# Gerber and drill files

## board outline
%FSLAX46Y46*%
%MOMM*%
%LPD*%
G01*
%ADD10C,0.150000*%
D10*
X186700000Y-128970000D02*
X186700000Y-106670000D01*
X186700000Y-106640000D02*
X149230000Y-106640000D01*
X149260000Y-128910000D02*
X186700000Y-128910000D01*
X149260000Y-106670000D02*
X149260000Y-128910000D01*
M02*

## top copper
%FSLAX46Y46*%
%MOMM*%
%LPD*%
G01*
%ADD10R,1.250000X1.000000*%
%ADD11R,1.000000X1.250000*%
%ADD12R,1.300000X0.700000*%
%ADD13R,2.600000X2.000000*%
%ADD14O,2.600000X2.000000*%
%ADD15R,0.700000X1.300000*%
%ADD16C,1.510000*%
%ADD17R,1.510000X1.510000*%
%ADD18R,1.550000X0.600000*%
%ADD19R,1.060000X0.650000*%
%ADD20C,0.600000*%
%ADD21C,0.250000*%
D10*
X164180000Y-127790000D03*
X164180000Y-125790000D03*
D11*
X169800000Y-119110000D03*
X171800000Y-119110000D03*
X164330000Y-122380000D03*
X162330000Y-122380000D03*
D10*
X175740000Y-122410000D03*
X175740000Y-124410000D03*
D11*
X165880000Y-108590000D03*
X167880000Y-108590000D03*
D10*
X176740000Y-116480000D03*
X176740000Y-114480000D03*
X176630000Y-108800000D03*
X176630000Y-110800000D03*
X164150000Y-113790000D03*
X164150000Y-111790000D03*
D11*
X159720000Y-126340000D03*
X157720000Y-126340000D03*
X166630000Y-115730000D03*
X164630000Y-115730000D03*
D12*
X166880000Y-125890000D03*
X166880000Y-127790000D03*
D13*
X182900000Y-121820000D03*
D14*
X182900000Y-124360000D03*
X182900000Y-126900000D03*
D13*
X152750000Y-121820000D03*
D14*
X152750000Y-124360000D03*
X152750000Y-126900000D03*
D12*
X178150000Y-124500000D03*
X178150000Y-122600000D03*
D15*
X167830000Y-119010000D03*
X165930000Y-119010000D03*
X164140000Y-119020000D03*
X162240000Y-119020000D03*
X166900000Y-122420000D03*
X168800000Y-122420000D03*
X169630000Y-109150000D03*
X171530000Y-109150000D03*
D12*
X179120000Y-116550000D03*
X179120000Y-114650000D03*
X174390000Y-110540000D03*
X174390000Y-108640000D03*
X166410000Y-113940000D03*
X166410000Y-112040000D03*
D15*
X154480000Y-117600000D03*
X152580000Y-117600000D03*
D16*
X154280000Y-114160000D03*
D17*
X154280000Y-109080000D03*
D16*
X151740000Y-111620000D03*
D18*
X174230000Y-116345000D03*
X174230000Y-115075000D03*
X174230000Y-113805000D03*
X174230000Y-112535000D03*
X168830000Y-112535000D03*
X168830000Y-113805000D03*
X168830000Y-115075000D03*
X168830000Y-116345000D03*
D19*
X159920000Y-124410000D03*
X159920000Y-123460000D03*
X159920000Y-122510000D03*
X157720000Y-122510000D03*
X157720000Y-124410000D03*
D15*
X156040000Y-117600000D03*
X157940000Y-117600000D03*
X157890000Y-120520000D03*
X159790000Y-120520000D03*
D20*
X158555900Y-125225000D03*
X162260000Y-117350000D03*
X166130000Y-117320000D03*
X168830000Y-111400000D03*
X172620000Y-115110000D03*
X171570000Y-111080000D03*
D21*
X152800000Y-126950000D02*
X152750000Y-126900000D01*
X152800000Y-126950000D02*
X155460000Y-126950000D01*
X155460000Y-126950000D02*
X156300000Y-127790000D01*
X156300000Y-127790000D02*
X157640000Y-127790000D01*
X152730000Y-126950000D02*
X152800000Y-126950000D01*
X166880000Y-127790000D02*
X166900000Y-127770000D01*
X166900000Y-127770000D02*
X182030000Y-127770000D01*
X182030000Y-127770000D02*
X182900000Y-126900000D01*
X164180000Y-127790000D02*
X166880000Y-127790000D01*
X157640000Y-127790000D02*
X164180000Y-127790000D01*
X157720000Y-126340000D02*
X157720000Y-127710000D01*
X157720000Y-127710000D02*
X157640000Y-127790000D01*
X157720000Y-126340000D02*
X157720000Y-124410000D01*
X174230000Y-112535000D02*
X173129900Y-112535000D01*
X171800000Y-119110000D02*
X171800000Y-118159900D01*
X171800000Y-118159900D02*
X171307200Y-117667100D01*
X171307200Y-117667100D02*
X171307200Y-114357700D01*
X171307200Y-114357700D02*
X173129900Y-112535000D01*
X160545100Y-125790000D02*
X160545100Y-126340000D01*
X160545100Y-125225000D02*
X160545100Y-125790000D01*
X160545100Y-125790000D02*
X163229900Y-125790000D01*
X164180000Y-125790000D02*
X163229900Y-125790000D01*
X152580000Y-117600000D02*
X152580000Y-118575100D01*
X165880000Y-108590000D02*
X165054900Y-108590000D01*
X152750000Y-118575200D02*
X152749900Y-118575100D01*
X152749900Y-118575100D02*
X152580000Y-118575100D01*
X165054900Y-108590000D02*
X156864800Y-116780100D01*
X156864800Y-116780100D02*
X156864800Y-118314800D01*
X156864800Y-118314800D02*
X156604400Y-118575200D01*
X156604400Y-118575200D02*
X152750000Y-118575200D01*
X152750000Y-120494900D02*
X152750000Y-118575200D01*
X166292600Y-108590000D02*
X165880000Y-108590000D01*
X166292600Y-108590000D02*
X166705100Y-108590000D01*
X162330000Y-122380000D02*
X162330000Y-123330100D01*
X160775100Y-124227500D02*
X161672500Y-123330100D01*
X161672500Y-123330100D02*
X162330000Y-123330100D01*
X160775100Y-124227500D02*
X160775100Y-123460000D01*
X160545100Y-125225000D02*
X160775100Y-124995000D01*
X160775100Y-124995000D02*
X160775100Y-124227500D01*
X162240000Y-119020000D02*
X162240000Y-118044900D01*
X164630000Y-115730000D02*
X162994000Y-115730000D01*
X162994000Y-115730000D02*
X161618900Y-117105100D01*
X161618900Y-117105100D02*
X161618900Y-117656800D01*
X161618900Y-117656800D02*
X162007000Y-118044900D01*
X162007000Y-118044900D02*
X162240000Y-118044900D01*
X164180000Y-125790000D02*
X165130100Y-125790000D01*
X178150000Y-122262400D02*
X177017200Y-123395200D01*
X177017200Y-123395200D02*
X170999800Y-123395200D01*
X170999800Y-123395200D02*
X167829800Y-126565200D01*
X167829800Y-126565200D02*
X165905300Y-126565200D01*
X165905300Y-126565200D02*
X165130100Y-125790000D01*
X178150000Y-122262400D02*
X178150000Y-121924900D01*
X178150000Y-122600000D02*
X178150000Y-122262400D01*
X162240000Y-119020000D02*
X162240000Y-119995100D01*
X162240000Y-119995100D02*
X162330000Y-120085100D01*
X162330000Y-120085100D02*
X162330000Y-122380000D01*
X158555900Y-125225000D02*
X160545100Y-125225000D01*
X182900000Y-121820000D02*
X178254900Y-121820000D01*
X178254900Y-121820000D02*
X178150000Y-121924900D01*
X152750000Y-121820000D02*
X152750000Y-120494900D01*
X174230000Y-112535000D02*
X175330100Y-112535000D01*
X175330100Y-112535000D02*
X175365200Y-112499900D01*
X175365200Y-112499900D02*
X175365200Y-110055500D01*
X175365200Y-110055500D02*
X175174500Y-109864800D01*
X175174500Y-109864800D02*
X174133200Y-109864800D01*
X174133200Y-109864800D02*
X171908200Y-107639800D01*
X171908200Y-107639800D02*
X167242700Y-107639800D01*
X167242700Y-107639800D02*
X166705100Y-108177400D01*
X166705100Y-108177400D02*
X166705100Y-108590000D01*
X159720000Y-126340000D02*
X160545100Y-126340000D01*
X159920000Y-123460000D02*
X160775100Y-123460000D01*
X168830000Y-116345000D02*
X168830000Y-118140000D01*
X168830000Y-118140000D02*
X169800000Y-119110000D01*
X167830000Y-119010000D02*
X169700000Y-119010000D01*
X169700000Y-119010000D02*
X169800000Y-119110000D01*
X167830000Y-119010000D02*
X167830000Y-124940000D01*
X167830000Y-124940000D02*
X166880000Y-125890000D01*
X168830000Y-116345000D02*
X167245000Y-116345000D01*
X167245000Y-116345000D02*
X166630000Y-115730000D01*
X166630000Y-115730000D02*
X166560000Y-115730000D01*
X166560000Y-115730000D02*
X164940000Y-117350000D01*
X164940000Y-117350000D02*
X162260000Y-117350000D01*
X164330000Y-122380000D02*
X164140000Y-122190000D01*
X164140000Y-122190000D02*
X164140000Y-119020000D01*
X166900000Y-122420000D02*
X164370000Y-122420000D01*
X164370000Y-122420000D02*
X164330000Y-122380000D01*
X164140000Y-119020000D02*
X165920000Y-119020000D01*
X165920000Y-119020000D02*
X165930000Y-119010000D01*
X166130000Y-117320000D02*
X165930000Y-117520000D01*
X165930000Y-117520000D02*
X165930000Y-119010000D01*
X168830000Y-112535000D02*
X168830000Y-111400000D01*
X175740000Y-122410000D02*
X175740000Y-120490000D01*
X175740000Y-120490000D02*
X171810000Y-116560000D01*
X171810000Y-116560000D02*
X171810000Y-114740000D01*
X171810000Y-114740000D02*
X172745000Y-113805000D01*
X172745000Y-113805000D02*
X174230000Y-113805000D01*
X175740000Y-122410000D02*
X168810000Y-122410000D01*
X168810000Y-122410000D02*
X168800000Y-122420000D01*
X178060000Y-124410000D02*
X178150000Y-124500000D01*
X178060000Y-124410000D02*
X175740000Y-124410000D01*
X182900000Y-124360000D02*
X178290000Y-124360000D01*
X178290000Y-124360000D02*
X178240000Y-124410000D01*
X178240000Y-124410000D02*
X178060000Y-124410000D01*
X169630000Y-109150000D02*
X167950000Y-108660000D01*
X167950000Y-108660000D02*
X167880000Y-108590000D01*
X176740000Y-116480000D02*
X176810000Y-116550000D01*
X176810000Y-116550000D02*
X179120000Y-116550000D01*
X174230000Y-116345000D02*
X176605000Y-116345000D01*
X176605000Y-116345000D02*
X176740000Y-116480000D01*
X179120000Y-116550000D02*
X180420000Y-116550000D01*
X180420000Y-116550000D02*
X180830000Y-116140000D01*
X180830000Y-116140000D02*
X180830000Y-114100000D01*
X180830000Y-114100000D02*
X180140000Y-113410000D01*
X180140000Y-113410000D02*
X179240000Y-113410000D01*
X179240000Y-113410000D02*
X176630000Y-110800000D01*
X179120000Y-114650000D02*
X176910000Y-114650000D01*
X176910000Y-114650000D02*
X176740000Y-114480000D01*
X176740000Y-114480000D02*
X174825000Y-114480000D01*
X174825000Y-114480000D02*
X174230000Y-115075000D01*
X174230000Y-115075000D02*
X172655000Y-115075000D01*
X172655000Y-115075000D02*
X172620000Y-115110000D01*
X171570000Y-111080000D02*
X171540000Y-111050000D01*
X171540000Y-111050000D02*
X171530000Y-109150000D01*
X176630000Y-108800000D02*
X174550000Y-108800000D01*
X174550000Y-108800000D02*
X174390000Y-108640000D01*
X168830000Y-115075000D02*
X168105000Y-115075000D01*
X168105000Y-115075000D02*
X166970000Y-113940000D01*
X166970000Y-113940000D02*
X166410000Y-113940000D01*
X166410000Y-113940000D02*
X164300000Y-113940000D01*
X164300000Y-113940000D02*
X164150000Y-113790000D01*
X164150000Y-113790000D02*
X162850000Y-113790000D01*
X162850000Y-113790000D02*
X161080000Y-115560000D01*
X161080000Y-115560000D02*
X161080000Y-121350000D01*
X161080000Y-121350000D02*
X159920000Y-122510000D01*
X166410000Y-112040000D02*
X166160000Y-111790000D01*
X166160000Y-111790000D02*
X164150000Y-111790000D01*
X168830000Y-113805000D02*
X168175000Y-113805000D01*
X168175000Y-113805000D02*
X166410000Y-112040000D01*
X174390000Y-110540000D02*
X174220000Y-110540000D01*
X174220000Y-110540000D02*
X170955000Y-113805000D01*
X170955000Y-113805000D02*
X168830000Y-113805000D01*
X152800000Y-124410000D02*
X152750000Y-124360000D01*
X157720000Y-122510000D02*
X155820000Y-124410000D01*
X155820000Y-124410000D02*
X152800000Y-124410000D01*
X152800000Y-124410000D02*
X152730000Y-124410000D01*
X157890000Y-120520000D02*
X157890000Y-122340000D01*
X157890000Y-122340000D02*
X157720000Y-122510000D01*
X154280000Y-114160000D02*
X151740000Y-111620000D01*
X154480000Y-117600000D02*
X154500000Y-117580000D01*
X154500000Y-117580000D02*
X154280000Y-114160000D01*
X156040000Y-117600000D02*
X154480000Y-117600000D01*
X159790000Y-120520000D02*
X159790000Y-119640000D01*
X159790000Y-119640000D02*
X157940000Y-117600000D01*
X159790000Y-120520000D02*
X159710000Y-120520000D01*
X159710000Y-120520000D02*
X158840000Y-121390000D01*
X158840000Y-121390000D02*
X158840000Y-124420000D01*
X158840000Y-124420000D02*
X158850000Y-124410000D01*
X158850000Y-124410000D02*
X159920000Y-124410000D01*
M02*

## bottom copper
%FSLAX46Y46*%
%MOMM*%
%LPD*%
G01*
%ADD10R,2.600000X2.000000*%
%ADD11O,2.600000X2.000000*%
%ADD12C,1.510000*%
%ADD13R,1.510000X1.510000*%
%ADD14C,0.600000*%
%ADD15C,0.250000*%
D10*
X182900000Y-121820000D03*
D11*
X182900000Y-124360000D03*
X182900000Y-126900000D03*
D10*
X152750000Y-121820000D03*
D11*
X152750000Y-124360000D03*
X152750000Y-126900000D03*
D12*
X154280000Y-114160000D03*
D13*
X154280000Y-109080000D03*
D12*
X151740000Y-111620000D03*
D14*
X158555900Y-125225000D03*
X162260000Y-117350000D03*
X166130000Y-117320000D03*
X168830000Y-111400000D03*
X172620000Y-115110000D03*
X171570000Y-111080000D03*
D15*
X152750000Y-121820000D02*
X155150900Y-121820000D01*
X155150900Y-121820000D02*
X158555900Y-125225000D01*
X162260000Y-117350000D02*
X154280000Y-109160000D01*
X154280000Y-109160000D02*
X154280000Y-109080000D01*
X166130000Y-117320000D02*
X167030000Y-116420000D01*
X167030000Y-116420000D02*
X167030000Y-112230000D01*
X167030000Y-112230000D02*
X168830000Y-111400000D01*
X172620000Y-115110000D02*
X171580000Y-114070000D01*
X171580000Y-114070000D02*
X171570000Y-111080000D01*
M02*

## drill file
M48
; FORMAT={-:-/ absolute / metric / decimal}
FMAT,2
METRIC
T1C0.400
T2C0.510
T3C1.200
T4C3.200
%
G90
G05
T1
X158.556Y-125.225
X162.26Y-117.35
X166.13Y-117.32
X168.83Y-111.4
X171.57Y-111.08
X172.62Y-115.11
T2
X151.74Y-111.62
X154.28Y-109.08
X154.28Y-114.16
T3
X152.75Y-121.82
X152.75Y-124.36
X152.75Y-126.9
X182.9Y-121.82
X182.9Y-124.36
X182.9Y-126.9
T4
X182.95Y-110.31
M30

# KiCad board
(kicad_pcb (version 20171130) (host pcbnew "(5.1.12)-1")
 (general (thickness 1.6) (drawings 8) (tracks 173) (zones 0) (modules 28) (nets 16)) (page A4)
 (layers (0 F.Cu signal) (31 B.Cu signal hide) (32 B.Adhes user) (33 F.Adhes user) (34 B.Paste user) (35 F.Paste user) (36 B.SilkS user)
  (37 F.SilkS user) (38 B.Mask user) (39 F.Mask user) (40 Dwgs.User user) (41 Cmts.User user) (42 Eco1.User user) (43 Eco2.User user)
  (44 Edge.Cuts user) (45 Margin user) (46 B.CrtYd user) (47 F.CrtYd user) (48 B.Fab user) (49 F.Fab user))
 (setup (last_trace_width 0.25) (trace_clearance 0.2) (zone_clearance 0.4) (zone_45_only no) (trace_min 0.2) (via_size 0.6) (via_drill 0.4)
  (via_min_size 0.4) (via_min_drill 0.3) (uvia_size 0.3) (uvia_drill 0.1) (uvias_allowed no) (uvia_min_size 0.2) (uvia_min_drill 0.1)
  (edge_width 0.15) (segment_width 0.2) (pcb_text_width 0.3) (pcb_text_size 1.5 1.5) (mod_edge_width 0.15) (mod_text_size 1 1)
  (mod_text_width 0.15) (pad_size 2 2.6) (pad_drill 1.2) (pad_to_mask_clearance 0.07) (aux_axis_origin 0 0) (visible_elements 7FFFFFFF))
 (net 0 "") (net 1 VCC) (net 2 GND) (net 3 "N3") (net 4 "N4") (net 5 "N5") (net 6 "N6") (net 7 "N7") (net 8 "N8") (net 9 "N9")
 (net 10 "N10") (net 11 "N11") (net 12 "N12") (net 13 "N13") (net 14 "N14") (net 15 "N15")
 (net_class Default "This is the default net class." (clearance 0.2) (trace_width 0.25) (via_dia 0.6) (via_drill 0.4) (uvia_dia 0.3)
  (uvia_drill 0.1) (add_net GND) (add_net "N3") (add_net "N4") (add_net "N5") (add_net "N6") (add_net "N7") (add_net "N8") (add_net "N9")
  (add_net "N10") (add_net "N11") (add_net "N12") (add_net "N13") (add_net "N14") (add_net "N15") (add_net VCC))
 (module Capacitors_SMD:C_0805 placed (layer F.Cu) (at 164.18 126.79 90)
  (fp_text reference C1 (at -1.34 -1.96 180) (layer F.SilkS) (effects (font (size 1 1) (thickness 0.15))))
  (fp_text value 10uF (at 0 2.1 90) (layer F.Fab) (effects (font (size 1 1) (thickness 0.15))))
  (pad 1 smd rect (at -1 0 90) (size 1 1.25) (layers F.Cu F.Paste F.Mask) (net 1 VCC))
  (pad 2 smd rect (at 1 0 90) (size 1 1.25) (layers F.Cu F.Paste F.Mask) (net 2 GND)))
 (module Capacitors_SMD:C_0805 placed (layer F.Cu) (at 170.8 119.11)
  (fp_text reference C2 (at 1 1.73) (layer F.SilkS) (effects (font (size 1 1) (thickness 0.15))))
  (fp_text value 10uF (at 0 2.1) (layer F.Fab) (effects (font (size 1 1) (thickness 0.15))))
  (pad 1 smd rect (at -1 0) (size 1 1.25) (layers F.Cu F.Paste F.Mask) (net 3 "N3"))
  (pad 2 smd rect (at 1 0) (size 1 1.25) (layers F.Cu F.Paste F.Mask) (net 2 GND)))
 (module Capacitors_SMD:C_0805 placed (layer F.Cu) (at 163.33 122.38 180)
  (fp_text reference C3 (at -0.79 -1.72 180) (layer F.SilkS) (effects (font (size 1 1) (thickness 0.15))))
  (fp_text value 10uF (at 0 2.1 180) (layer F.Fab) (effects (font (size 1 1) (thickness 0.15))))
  (pad 1 smd rect (at -1 0 180) (size 1 1.25) (layers F.Cu F.Paste F.Mask) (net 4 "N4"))
  (pad 2 smd rect (at 1 0 180) (size 1 1.25) (layers F.Cu F.Paste F.Mask) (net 2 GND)))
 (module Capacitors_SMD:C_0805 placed (layer F.Cu) (at 175.74 123.41 270)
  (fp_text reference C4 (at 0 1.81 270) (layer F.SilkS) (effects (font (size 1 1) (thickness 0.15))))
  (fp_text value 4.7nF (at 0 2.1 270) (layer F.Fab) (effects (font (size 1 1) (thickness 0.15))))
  (pad 1 smd rect (at -1 0 270) (size 1 1.25) (layers F.Cu F.Paste F.Mask) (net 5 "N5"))
  (pad 2 smd rect (at 1 0 270) (size 1 1.25) (layers F.Cu F.Paste F.Mask) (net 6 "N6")))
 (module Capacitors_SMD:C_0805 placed (layer F.Cu) (at 166.88 108.59)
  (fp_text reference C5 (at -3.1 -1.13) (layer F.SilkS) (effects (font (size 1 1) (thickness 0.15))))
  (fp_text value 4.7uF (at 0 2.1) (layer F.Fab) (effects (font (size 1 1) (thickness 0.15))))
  (pad 1 smd rect (at -1 0) (size 1 1.25) (layers F.Cu F.Paste F.Mask) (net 2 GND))
  (pad 2 smd rect (at 1 0) (size 1 1.25) (layers F.Cu F.Paste F.Mask) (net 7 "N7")))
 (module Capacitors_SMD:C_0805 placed (layer F.Cu) (at 176.74 115.48 90)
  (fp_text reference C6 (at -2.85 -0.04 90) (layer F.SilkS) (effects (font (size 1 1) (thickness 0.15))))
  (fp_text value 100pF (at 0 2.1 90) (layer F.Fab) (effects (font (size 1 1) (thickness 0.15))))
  (pad 1 smd rect (at -1 0 90) (size 1 1.25) (layers F.Cu F.Paste F.Mask) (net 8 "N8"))
  (pad 2 smd rect (at 1 0 90) (size 1 1.25) (layers F.Cu F.Paste F.Mask) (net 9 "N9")))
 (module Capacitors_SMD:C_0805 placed (layer F.Cu) (at 176.63 109.8 270)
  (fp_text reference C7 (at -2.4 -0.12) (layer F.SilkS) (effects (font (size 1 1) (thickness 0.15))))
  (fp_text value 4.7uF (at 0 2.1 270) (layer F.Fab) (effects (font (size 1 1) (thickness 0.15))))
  (pad 1 smd rect (at -1 0 270) (size 1 1.25) (layers F.Cu F.Paste F.Mask) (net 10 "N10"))
  (pad 2 smd rect (at 1 0 270) (size 1 1.25) (layers F.Cu F.Paste F.Mask) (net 8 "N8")))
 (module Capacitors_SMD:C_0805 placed (layer F.Cu) (at 164.15 112.79 90)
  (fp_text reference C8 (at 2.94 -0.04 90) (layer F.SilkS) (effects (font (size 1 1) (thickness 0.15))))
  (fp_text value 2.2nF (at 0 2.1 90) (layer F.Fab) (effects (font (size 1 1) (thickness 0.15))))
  (pad 1 smd rect (at -1 0 90) (size 1 1.25) (layers F.Cu F.Paste F.Mask) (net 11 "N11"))
  (pad 2 smd rect (at 1 0 90) (size 1 1.25) (layers F.Cu F.Paste F.Mask) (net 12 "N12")))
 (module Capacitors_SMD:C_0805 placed (layer F.Cu) (at 158.72 126.34 180)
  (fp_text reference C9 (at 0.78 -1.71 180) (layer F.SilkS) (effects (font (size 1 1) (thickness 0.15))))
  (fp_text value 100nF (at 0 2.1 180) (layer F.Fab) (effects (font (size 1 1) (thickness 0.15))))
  (pad 1 smd rect (at -1 0 180) (size 1 1.25) (layers F.Cu F.Paste F.Mask) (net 2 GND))
  (pad 2 smd rect (at 1 0 180) (size 1 1.25) (layers F.Cu F.Paste F.Mask) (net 1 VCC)))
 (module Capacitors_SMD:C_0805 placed (layer F.Cu) (at 165.63 115.73 180)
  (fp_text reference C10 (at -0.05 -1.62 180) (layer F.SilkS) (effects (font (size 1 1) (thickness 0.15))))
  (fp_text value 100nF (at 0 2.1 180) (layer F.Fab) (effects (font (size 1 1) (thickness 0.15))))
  (pad 1 smd rect (at -1 0 180) (size 1 1.25) (layers F.Cu F.Paste F.Mask) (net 3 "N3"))
  (pad 2 smd rect (at 1 0 180) (size 1 1.25) (layers F.Cu F.Paste F.Mask) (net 2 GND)))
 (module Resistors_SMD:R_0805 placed (layer F.Cu) (at 166.88 126.84 270)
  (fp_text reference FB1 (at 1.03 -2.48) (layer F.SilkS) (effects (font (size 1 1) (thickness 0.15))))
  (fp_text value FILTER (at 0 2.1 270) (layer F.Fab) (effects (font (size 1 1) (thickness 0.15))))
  (pad 1 smd rect (at -0.95 0 270) (size 0.7 1.3) (layers F.Cu F.Paste F.Mask) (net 3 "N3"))
  (pad 2 smd rect (at 0.95 0 270) (size 0.7 1.3) (layers F.Cu F.Paste F.Mask) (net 1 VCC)))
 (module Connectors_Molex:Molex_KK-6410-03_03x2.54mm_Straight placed (layer F.Cu) (at 182.9 121.82 270)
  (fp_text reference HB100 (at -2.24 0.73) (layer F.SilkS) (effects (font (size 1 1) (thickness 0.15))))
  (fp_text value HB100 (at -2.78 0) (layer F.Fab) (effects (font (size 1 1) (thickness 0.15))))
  (pad 1 thru_hole rect (at 0 0 270) (size 2 2.6) (drill 1.2) (layers *.Cu *.Mask F.SilkS) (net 2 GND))
  (pad 2 thru_hole oval (at 2.54 0 270) (size 2 2.6) (drill 1.2) (layers *.Cu *.Mask F.SilkS) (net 6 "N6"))
  (pad 3 thru_hole oval (at 5.08 0 270) (size 2 2.6) (drill 1.2) (layers *.Cu *.Mask F.SilkS) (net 1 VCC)))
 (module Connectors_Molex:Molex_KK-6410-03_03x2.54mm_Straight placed (layer F.Cu) (at 152.75 121.82 270)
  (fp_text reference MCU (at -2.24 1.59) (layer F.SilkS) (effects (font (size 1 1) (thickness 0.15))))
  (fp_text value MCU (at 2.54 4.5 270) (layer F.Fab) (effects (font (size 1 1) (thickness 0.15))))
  (pad 3 thru_hole rect (at 0 0 270) (size 2 2.6) (drill 1.2) (layers *.Cu *.Mask F.SilkS) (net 2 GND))
  (pad 2 thru_hole oval (at 2.54 0 270) (size 2 2.6) (drill 1.2) (layers *.Cu *.Mask F.SilkS) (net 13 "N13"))
  (pad 1 thru_hole oval (at 5.08 0 270) (size 2 2.6) (drill 1.2) (layers *.Cu *.Mask F.SilkS) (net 1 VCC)))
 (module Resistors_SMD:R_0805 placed (layer F.Cu) (at 178.15 123.55 90)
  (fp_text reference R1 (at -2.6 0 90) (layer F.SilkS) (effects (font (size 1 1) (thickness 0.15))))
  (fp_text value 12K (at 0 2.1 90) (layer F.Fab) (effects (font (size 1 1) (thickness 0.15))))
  (pad 1 smd rect (at -0.95 0 90) (size 0.7 1.3) (layers F.Cu F.Paste F.Mask) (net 6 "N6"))
  (pad 2 smd rect (at 0.95 0 90) (size 0.7 1.3) (layers F.Cu F.Paste F.Mask) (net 2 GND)))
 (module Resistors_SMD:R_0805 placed (layer F.Cu) (at 166.88 119.01 180)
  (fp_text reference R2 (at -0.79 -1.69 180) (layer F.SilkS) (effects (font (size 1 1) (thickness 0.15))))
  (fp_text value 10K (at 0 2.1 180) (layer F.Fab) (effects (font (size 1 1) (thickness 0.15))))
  (pad 1 smd rect (at -0.95 0 180) (size 0.7 1.3) (layers F.Cu F.Paste F.Mask) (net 3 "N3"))
  (pad 2 smd rect (at 0.95 0 180) (size 0.7 1.3) (layers F.Cu F.Paste F.Mask) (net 4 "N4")))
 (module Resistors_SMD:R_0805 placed (layer F.Cu) (at 163.19 119.02 180)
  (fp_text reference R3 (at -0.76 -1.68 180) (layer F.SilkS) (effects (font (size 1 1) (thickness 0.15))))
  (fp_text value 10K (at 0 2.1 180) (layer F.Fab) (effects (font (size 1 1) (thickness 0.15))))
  (pad 1 smd rect (at -0.95 0 180) (size 0.7 1.3) (layers F.Cu F.Paste F.Mask) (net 4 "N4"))
  (pad 2 smd rect (at 0.95 0 180) (size 0.7 1.3) (layers F.Cu F.Paste F.Mask) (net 2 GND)))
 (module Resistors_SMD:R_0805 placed (layer F.Cu) (at 167.85 122.42)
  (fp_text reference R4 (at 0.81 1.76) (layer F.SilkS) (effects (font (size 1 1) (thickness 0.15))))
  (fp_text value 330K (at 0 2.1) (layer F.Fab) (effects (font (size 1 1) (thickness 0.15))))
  (pad 1 smd rect (at -0.95 0) (size 0.7 1.3) (layers F.Cu F.Paste F.Mask) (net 4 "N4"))
  (pad 2 smd rect (at 0.95 0) (size 0.7 1.3) (layers F.Cu F.Paste F.Mask) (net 5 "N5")))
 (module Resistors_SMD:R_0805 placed (layer F.Cu) (at 170.58 109.15)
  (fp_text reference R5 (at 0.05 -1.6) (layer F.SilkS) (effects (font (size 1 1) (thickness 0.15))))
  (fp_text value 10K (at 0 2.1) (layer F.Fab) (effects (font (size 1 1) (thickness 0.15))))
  (pad 1 smd rect (at -0.95 0) (size 0.7 1.3) (layers F.Cu F.Paste F.Mask) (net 7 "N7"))
  (pad 2 smd rect (at 0.95 0) (size 0.7 1.3) (layers F.Cu F.Paste F.Mask) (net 9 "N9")))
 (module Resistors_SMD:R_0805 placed (layer F.Cu) (at 179.12 115.6 90)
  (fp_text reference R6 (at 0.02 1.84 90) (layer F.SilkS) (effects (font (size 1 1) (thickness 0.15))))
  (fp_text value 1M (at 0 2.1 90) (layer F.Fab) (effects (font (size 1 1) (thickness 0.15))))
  (pad 1 smd rect (at -0.95 0 90) (size 0.7 1.3) (layers F.Cu F.Paste F.Mask) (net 8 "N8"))
  (pad 2 smd rect (at 0.95 0 90) (size 0.7 1.3) (layers F.Cu F.Paste F.Mask) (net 9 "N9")))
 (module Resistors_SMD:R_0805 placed (layer F.Cu) (at 174.39 109.59 90)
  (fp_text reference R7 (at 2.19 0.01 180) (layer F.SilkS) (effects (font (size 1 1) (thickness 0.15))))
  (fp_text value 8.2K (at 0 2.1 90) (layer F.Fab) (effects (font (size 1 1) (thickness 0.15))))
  (pad 1 smd rect (at -0.95 0 90) (size 0.7 1.3) (layers F.Cu F.Paste F.Mask) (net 12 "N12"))
  (pad 2 smd rect (at 0.95 0 90) (size 0.7 1.3) (layers F.Cu F.Paste F.Mask) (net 10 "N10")))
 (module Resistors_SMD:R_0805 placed (layer F.Cu) (at 166.41 112.99 90)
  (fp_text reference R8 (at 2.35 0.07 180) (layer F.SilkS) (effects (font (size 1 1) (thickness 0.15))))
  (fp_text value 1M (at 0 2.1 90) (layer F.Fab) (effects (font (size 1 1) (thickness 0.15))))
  (pad 1 smd rect (at -0.95 0 90) (size 0.7 1.3) (layers F.Cu F.Paste F.Mask) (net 11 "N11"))
  (pad 2 smd rect (at 0.95 0 90) (size 0.7 1.3) (layers F.Cu F.Paste F.Mask) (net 12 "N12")))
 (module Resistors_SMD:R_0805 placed (layer F.Cu) (at 153.53 117.6 180)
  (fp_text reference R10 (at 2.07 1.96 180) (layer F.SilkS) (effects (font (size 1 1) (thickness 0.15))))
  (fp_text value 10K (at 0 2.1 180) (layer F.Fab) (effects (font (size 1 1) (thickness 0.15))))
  (pad 1 smd rect (at -0.95 0 180) (size 0.7 1.3) (layers F.Cu F.Paste F.Mask) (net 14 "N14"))
  (pad 2 smd rect (at 0.95 0 180) (size 0.7 1.3) (layers F.Cu F.Paste F.Mask) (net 2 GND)))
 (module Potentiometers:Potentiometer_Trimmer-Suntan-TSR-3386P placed (layer F.Cu) (at 154.28 109.08 270)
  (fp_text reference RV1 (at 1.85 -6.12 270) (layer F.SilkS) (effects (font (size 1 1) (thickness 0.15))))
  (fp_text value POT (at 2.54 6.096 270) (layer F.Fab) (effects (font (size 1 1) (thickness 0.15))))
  (pad 3 thru_hole circle (at 5.08 0 270) (size 1.51 1.51) (drill 0.51) (layers *.Cu *.Mask F.SilkS) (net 14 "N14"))
  (pad 1 thru_hole rect (at 0 0 270) (size 1.51 1.51) (drill 0.51) (layers *.Cu *.Mask F.SilkS) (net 3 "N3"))
  (pad 2 thru_hole circle (at 2.54 2.54 270) (size 1.51 1.51) (drill 0.51) (layers *.Cu *.Mask F.SilkS) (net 14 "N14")))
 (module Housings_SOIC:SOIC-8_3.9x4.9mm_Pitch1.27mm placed (layer F.Cu) (at 171.53 114.44 180)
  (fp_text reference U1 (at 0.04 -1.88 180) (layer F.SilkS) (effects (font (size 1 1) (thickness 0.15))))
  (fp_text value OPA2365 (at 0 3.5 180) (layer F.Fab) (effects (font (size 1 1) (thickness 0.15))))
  (pad 1 smd rect (at -2.7 -1.905 180) (size 1.55 0.6) (layers F.Cu F.Paste F.Mask) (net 8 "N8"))
  (pad 2 smd rect (at -2.7 -0.635 180) (size 1.55 0.6) (layers F.Cu F.Paste F.Mask) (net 9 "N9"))
  (pad 3 smd rect (at -2.7 0.635 180) (size 1.55 0.6) (layers F.Cu F.Paste F.Mask) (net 5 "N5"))
  (pad 4 smd rect (at -2.7 1.905 180) (size 1.55 0.6) (layers F.Cu F.Paste F.Mask) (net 2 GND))
  (pad 5 smd rect (at 2.7 1.905 180) (size 1.55 0.6) (layers F.Cu F.Paste F.Mask) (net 4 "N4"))
  (pad 6 smd rect (at 2.7 0.635 180) (size 1.55 0.6) (layers F.Cu F.Paste F.Mask) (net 12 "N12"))
  (pad 7 smd rect (at 2.7 -0.635 180) (size 1.55 0.6) (layers F.Cu F.Paste F.Mask) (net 11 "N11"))
  (pad 8 smd rect (at 2.7 -1.905 180) (size 1.55 0.6) (layers F.Cu F.Paste F.Mask) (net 3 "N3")))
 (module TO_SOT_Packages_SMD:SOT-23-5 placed (layer F.Cu) (at 158.82 123.46 180)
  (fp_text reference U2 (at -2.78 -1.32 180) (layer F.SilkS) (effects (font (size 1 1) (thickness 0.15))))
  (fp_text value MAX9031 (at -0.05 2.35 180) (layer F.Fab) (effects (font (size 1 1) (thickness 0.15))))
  (pad 1 smd rect (at -1.1 -0.95 180) (size 1.06 0.65) (layers F.Cu F.Paste F.Mask) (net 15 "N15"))
  (pad 2 smd rect (at -1.1 0 180) (size 1.06 0.65) (layers F.Cu F.Paste F.Mask) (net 2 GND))
  (pad 3 smd rect (at -1.1 0.95 180) (size 1.06 0.65) (layers F.Cu F.Paste F.Mask) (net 11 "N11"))
  (pad 4 smd rect (at 1.1 0.95 180) (size 1.06 0.65) (layers F.Cu F.Paste F.Mask) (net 13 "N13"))
  (pad 5 smd rect (at 1.1 -0.95 180) (size 1.06 0.65) (layers F.Cu F.Paste F.Mask) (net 1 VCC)))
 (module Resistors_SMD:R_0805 (layer F.Cu) (at 156.99 117.6)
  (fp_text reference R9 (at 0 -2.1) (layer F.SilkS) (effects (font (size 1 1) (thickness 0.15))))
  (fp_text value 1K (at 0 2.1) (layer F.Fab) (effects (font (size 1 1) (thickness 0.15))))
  (pad 1 smd rect (at -0.95 0) (size 0.7 1.3) (layers F.Cu F.Paste F.Mask) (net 14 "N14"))
  (pad 2 smd rect (at 0.95 0) (size 0.7 1.3) (layers F.Cu F.Paste F.Mask) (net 15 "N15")))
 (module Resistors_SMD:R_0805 (layer F.Cu) (at 158.84 120.52)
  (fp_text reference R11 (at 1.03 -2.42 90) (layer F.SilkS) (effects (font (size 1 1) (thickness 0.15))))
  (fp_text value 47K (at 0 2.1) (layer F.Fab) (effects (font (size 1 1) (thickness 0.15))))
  (pad 1 smd rect (at -0.95 0) (size 0.7 1.3) (layers F.Cu F.Paste F.Mask) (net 13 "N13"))
  (pad 2 smd rect (at 0.95 0) (size 0.7 1.3) (layers F.Cu F.Paste F.Mask) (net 15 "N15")))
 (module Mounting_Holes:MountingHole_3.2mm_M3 (layer F.Cu) (at 182.95 110.31)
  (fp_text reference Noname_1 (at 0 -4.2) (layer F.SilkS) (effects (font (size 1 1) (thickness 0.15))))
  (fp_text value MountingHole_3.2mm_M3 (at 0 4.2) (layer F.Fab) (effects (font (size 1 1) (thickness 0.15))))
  (pad 1 np_thru_hole circle (at 0 0) (size 3.2 3.2) (drill 3.2) (layers *.Cu *.Mask F.SilkS)))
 (gr_line (start 186.7 128.97) (end 186.7 106.67) (angle 90) (layer Edge.Cuts) (width 0.15))
 (gr_line (start 186.7 106.64) (end 149.23 106.64) (angle 90) (layer Edge.Cuts) (width 0.15))
 (gr_line (start 149.26 128.91) (end 186.7 128.91) (angle 90) (layer Edge.Cuts) (width 0.15))
 (gr_line (start 149.26 106.67) (end 149.26 128.91) (angle 90) (layer Edge.Cuts) (width 0.15))
 (segment (start 152.8 126.95) (end 152.75 126.9) (width 0.25) (layer F.Cu) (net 1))
 (segment (start 152.8 126.95) (end 155.46 126.95) (width 0.25) (layer F.Cu) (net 1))
 (segment (start 155.46 126.95) (end 156.3 127.79) (width 0.25) (layer F.Cu) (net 1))
 (segment (start 156.3 127.79) (end 157.64 127.79) (width 0.25) (layer F.Cu) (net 1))
 (segment (start 152.73 126.95) (end 152.8 126.95) (width 0.25) (layer F.Cu) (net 1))
 (segment (start 166.88 127.79) (end 166.9 127.77) (width 0.25) (layer F.Cu) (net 1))
 (segment (start 166.9 127.77) (end 182.03 127.77) (width 0.25) (layer F.Cu) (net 1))
 (segment (start 182.03 127.77) (end 182.9 126.9) (width 0.25) (layer F.Cu) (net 1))
 (segment (start 164.18 127.79) (end 166.88 127.79) (width 0.25) (layer F.Cu) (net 1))
 (segment (start 157.64 127.79) (end 164.18 127.79) (width 0.25) (layer F.Cu) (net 1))
 (segment (start 157.72 126.34) (end 157.72 127.71) (width 0.25) (layer F.Cu) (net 1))
 (segment (start 157.72 127.71) (end 157.64 127.79) (width 0.25) (layer F.Cu) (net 1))
 (segment (start 157.72 126.34) (end 157.72 124.41) (width 0.25) (layer F.Cu) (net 1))
 (segment (start 174.23 112.535) (end 173.1299 112.535) (width 0.25) (layer F.Cu) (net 2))
 (segment (start 171.8 119.11) (end 171.8 118.1599) (width 0.25) (layer F.Cu) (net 2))
 (segment (start 171.8 118.1599) (end 171.3072 117.6671) (width 0.25) (layer F.Cu) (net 2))
 (segment (start 171.3072 117.6671) (end 171.3072 114.3577) (width 0.25) (layer F.Cu) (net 2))
 (segment (start 171.3072 114.3577) (end 173.1299 112.535) (width 0.25) (layer F.Cu) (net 2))
 (segment (start 160.5451 125.79) (end 160.5451 126.34) (width 0.25) (layer F.Cu) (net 2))
 (segment (start 160.5451 125.225) (end 160.5451 125.79) (width 0.25) (layer F.Cu) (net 2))
 (segment (start 160.5451 125.79) (end 163.2299 125.79) (width 0.25) (layer F.Cu) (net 2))
 (segment (start 164.18 125.79) (end 163.2299 125.79) (width 0.25) (layer F.Cu) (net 2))
 (segment (start 152.58 117.6) (end 152.58 118.5751) (width 0.25) (layer F.Cu) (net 2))
 (segment (start 165.88 108.59) (end 165.0549 108.59) (width 0.25) (layer F.Cu) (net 2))
 (segment (start 152.75 118.5752) (end 152.7499 118.5751) (width 0.25) (layer F.Cu) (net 2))
 (segment (start 152.7499 118.5751) (end 152.58 118.5751) (width 0.25) (layer F.Cu) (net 2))
 (segment (start 165.0549 108.59) (end 156.8648 116.7801) (width 0.25) (layer F.Cu) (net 2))
 (segment (start 156.8648 116.7801) (end 156.8648 118.3148) (width 0.25) (layer F.Cu) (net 2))
 (segment (start 156.8648 118.3148) (end 156.6044 118.5752) (width 0.25) (layer F.Cu) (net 2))
 (segment (start 156.6044 118.5752) (end 152.75 118.5752) (width 0.25) (layer F.Cu) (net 2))
 (segment (start 152.75 120.4949) (end 152.75 118.5752) (width 0.25) (layer F.Cu) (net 2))
 (segment (start 166.2926 108.59) (end 165.88 108.59) (width 0.25) (layer F.Cu) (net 2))
 (segment (start 166.2926 108.59) (end 166.7051 108.59) (width 0.25) (layer F.Cu) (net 2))
 (segment (start 162.33 122.38) (end 162.33 123.3301) (width 0.25) (layer F.Cu) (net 2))
 (segment (start 160.7751 124.2275) (end 161.6725 123.3301) (width 0.25) (layer F.Cu) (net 2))
 (segment (start 161.6725 123.3301) (end 162.33 123.3301) (width 0.25) (layer F.Cu) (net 2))
 (segment (start 160.7751 124.2275) (end 160.7751 123.46) (width 0.25) (layer F.Cu) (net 2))
 (segment (start 160.5451 125.225) (end 160.7751 124.995) (width 0.25) (layer F.Cu) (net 2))
 (segment (start 160.7751 124.995) (end 160.7751 124.2275) (width 0.25) (layer F.Cu) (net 2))
 (segment (start 162.24 119.02) (end 162.24 118.0449) (width 0.25) (layer F.Cu) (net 2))
 (segment (start 164.63 115.73) (end 162.994 115.73) (width 0.25) (layer F.Cu) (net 2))
 (segment (start 162.994 115.73) (end 161.6189 117.1051) (width 0.25) (layer F.Cu) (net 2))
 (segment (start 161.6189 117.1051) (end 161.6189 117.6568) (width 0.25) (layer F.Cu) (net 2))
 (segment (start 161.6189 117.6568) (end 162.007 118.0449) (width 0.25) (layer F.Cu) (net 2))
 (segment (start 162.007 118.0449) (end 162.24 118.0449) (width 0.25) (layer F.Cu) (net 2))
 (segment (start 164.18 125.79) (end 165.1301 125.79) (width 0.25) (layer F.Cu) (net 2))
 (segment (start 178.15 122.2624) (end 177.0172 123.3952) (width 0.25) (layer F.Cu) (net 2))
 (segment (start 177.0172 123.3952) (end 170.9998 123.3952) (width 0.25) (layer F.Cu) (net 2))
 (segment (start 170.9998 123.3952) (end 167.8298 126.5652) (width 0.25) (layer F.Cu) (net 2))
 (segment (start 167.8298 126.5652) (end 165.9053 126.5652) (width 0.25) (layer F.Cu) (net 2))
 (segment (start 165.9053 126.5652) (end 165.1301 125.79) (width 0.25) (layer F.Cu) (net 2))
 (segment (start 178.15 122.2624) (end 178.15 121.9249) (width 0.25) (layer F.Cu) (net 2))
 (segment (start 178.15 122.6) (end 178.15 122.2624) (width 0.25) (layer F.Cu) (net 2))
 (segment (start 162.24 119.02) (end 162.24 119.9951) (width 0.25) (layer F.Cu) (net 2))
 (segment (start 162.24 119.9951) (end 162.33 120.0851) (width 0.25) (layer F.Cu) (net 2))
 (segment (start 162.33 120.0851) (end 162.33 122.38) (width 0.25) (layer F.Cu) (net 2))
 (segment (start 158.5559 125.225) (end 160.5451 125.225) (width 0.25) (layer F.Cu) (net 2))
 (segment (start 152.75 121.82) (end 155.1509 121.82) (width 0.25) (layer B.Cu) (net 2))
 (segment (start 155.1509 121.82) (end 158.5559 125.225) (width 0.25) (layer B.Cu) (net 2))
 (segment (start 182.9 121.82) (end 178.2549 121.82) (width 0.25) (layer F.Cu) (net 2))
 (segment (start 178.2549 121.82) (end 178.15 121.9249) (width 0.25) (layer F.Cu) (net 2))
 (segment (start 152.75 121.82) (end 152.75 120.4949) (width 0.25) (layer F.Cu) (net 2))
 (segment (start 174.23 112.535) (end 175.3301 112.535) (width 0.25) (layer F.Cu) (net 2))
 (segment (start 175.3301 112.535) (end 175.3652 112.4999) (width 0.25) (layer F.Cu) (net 2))
 (segment (start 175.3652 112.4999) (end 175.3652 110.0555) (width 0.25) (layer F.Cu) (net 2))
 (segment (start 175.3652 110.0555) (end 175.1745 109.8648) (width 0.25) (layer F.Cu) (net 2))
 (segment (start 175.1745 109.8648) (end 174.1332 109.8648) (width 0.25) (layer F.Cu) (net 2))
 (segment (start 174.1332 109.8648) (end 171.9082 107.6398) (width 0.25) (layer F.Cu) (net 2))
 (segment (start 171.9082 107.6398) (end 167.2427 107.6398) (width 0.25) (layer F.Cu) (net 2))
 (segment (start 167.2427 107.6398) (end 166.7051 108.1774) (width 0.25) (layer F.Cu) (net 2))
 (segment (start 166.7051 108.1774) (end 166.7051 108.59) (width 0.25) (layer F.Cu) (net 2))
 (segment (start 159.72 126.34) (end 160.5451 126.34) (width 0.25) (layer F.Cu) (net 2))
 (segment (start 159.92 123.46) (end 160.7751 123.46) (width 0.25) (layer F.Cu) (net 2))
 (via (at 158.5559 125.225) (size 0.6) (layers F.Cu B.Cu) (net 2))
 (segment (start 168.83 116.345) (end 168.83 118.14) (width 0.25) (layer F.Cu) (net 3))
 (segment (start 168.83 118.14) (end 169.8 119.11) (width 0.25) (layer F.Cu) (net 3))
 (segment (start 167.83 119.01) (end 169.7 119.01) (width 0.25) (layer F.Cu) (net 3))
 (segment (start 169.7 119.01) (end 169.8 119.11) (width 0.25) (layer F.Cu) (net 3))
 (segment (start 167.83 119.01) (end 167.83 124.94) (width 0.25) (layer F.Cu) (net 3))
 (segment (start 167.83 124.94) (end 166.88 125.89) (width 0.25) (layer F.Cu) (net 3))
 (segment (start 168.83 116.345) (end 167.245 116.345) (width 0.25) (layer F.Cu) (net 3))
 (segment (start 167.245 116.345) (end 166.63 115.73) (width 0.25) (layer F.Cu) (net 3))
 (segment (start 162.26 117.35) (end 154.28 109.16) (width 0.25) (layer B.Cu) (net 3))
 (segment (start 154.28 109.16) (end 154.28 109.08) (width 0.25) (layer B.Cu) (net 3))
 (segment (start 166.63 115.73) (end 166.56 115.73) (width 0.25) (layer F.Cu) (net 3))
 (segment (start 166.56 115.73) (end 164.94 117.35) (width 0.25) (layer F.Cu) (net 3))
 (segment (start 164.94 117.35) (end 162.26 117.35) (width 0.25) (layer F.Cu) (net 3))
 (via (at 162.26 117.35) (size 0.6) (layers F.Cu B.Cu) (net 3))
 (segment (start 164.33 122.38) (end 164.14 122.19) (width 0.25) (layer F.Cu) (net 4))
 (segment (start 164.14 122.19) (end 164.14 119.02) (width 0.25) (layer F.Cu) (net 4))
 (segment (start 166.9 122.42) (end 164.37 122.42) (width 0.25) (layer F.Cu) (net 4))
 (segment (start 164.37 122.42) (end 164.33 122.38) (width 0.25) (layer F.Cu) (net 4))
 (segment (start 164.14 119.02) (end 165.92 119.02) (width 0.25) (layer F.Cu) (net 4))
 (segment (start 165.92 119.02) (end 165.93 119.01) (width 0.25) (layer F.Cu) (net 4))
 (segment (start 166.13 117.32) (end 165.93 117.52) (width 0.25) (layer F.Cu) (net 4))
 (segment (start 165.93 117.52) (end 165.93 119.01) (width 0.25) (layer F.Cu) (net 4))
 (segment (start 166.13 117.32) (end 167.03 116.42) (width 0.25) (layer B.Cu) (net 4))
 (segment (start 167.03 116.42) (end 167.03 112.23) (width 0.25) (layer B.Cu) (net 4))
 (segment (start 167.03 112.23) (end 168.83 111.4) (width 0.25) (layer B.Cu) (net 4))
 (segment (start 168.83 112.535) (end 168.83 111.4) (width 0.25) (layer F.Cu) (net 4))
 (via (at 166.13 117.32) (size 0.6) (layers F.Cu B.Cu) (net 4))
 (via (at 168.83 111.4) (size 0.6) (layers F.Cu B.Cu) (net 4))
 (segment (start 175.74 122.41) (end 175.74 120.49) (width 0.25) (layer F.Cu) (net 5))
 (segment (start 175.74 120.49) (end 171.81 116.56) (width 0.25) (layer F.Cu) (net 5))
 (segment (start 171.81 116.56) (end 171.81 114.74) (width 0.25) (layer F.Cu) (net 5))
 (segment (start 171.81 114.74) (end 172.745 113.805) (width 0.25) (layer F.Cu) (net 5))
 (segment (start 172.745 113.805) (end 174.23 113.805) (width 0.25) (layer F.Cu) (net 5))
 (segment (start 175.74 122.41) (end 168.81 122.41) (width 0.25) (layer F.Cu) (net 5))
 (segment (start 168.81 122.41) (end 168.8 122.42) (width 0.25) (layer F.Cu) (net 5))
 (segment (start 178.06 124.41) (end 178.15 124.5) (width 0.25) (layer F.Cu) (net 6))
 (segment (start 178.06 124.41) (end 175.74 124.41) (width 0.25) (layer F.Cu) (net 6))
 (segment (start 182.9 124.36) (end 178.29 124.36) (width 0.25) (layer F.Cu) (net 6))
 (segment (start 178.29 124.36) (end 178.24 124.41) (width 0.25) (layer F.Cu) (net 6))
 (segment (start 178.24 124.41) (end 178.06 124.41) (width 0.25) (layer F.Cu) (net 6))
 (segment (start 169.63 109.15) (end 167.95 108.66) (width 0.25) (layer F.Cu) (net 7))
 (segment (start 167.95 108.66) (end 167.88 108.59) (width 0.25) (layer F.Cu) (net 7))
 (segment (start 176.74 116.48) (end 176.81 116.55) (width 0.25) (layer F.Cu) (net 8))
 (segment (start 176.81 116.55) (end 179.12 116.55) (width 0.25) (layer F.Cu) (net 8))
 (segment (start 174.23 116.345) (end 176.605 116.345) (width 0.25) (layer F.Cu) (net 8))
 (segment (start 176.605 116.345) (end 176.74 116.48) (width 0.25) (layer F.Cu) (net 8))
 (segment (start 179.12 116.55) (end 180.42 116.55) (width 0.25) (layer F.Cu) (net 8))
 (segment (start 180.42 116.55) (end 180.83 116.14) (width 0.25) (layer F.Cu) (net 8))
 (segment (start 180.83 116.14) (end 180.83 114.1) (width 0.25) (layer F.Cu) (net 8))
 (segment (start 180.83 114.1) (end 180.14 113.41) (width 0.25) (layer F.Cu) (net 8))
 (segment (start 180.14 113.41) (end 179.24 113.41) (width 0.25) (layer F.Cu) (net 8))
 (segment (start 179.24 113.41) (end 176.63 110.8) (width 0.25) (layer F.Cu) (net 8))
 (segment (start 179.12 114.65) (end 176.91 114.65) (width 0.25) (layer F.Cu) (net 9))
 (segment (start 176.91 114.65) (end 176.74 114.48) (width 0.25) (layer F.Cu) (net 9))
 (segment (start 176.74 114.48) (end 174.825 114.48) (width 0.25) (layer F.Cu) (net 9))
 (segment (start 174.825 114.48) (end 174.23 115.075) (width 0.25) (layer F.Cu) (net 9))
 (segment (start 174.23 115.075) (end 172.655 115.075) (width 0.25) (layer F.Cu) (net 9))
 (segment (start 172.655 115.075) (end 172.62 115.11) (width 0.25) (layer F.Cu) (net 9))
 (segment (start 171.57 111.08) (end 171.54 111.05) (width 0.25) (layer F.Cu) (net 9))
 (segment (start 171.54 111.05) (end 171.53 109.15) (width 0.25) (layer F.Cu) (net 9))
 (segment (start 172.62 115.11) (end 171.58 114.07) (width 0.25) (layer B.Cu) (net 9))
 (segment (start 171.58 114.07) (end 171.57 111.08) (width 0.25) (layer B.Cu) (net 9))
 (via (at 172.62 115.11) (size 0.6) (layers F.Cu B.Cu) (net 9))
 (via (at 171.57 111.08) (size 0.6) (layers F.Cu B.Cu) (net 9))
 (segment (start 176.63 108.8) (end 174.55 108.8) (width 0.25) (layer F.Cu) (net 10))
 (segment (start 174.55 108.8) (end 174.39 108.64) (width 0.25) (layer F.Cu) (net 10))
 (segment (start 168.83 115.075) (end 168.105 115.075) (width 0.25) (layer F.Cu) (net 11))
 (segment (start 168.105 115.075) (end 166.97 113.94) (width 0.25) (layer F.Cu) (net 11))
 (segment (start 166.97 113.94) (end 166.41 113.94) (width 0.25) (layer F.Cu) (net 11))
 (segment (start 166.41 113.94) (end 164.3 113.94) (width 0.25) (layer F.Cu) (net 11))
 (segment (start 164.3 113.94) (end 164.15 113.79) (width 0.25) (layer F.Cu) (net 11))
 (segment (start 164.15 113.79) (end 162.85 113.79) (width 0.25) (layer F.Cu) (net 11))
 (segment (start 162.85 113.79) (end 161.08 115.56) (width 0.25) (layer F.Cu) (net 11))
 (segment (start 161.08 115.56) (end 161.08 121.35) (width 0.25) (layer F.Cu) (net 11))
 (segment (start 161.08 121.35) (end 159.92 122.51) (width 0.25) (layer F.Cu) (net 11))
 (segment (start 166.41 112.04) (end 166.16 111.79) (width 0.25) (layer F.Cu) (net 12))
 (segment (start 166.16 111.79) (end 164.15 111.79) (width 0.25) (layer F.Cu) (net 12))
 (segment (start 168.83 113.805) (end 168.175 113.805) (width 0.25) (layer F.Cu) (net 12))
 (segment (start 168.175 113.805) (end 166.41 112.04) (width 0.25) (layer F.Cu) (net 12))
 (segment (start 174.39 110.54) (end 174.22 110.54) (width 0.25) (layer F.Cu) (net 12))
 (segment (start 174.22 110.54) (end 170.955 113.805) (width 0.25) (layer F.Cu) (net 12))
 (segment (start 170.955 113.805) (end 168.83 113.805) (width 0.25) (layer F.Cu) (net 12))
 (segment (start 152.8 124.41) (end 152.75 124.36) (width 0.25) (layer F.Cu) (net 13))
 (segment (start 157.72 122.51) (end 155.82 124.41) (width 0.25) (layer F.Cu) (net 13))
 (segment (start 155.82 124.41) (end 152.8 124.41) (width 0.25) (layer F.Cu) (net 13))
 (segment (start 152.8 124.41) (end 152.73 124.41) (width 0.25) (layer F.Cu) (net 13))
 (segment (start 157.89 120.52) (end 157.89 122.34) (width 0.25) (layer F.Cu) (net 13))
 (segment (start 157.89 122.34) (end 157.72 122.51) (width 0.25) (layer F.Cu) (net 13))
 (segment (start 154.28 114.16) (end 151.74 111.62) (width 0.25) (layer F.Cu) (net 14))
 (segment (start 154.48 117.6) (end 154.5 117.58) (width 0.25) (layer F.Cu) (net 14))
 (segment (start 154.5 117.58) (end 154.28 114.16) (width 0.25) (layer F.Cu) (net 14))
 (segment (start 156.04 117.6) (end 154.48 117.6) (width 0.25) (layer F.Cu) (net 14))
 (segment (start 159.79 120.52) (end 159.79 119.64) (width 0.25) (layer F.Cu) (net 15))
 (segment (start 159.79 119.64) (end 157.94 117.6) (width 0.25) (layer F.Cu) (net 15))
 (segment (start 159.79 120.52) (end 159.71 120.52) (width 0.25) (layer F.Cu) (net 15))
 (segment (start 159.71 120.52) (end 158.84 121.39) (width 0.25) (layer F.Cu) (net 15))
 (segment (start 158.84 121.39) (end 158.84 124.42) (width 0.25) (layer F.Cu) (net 15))
 (segment (start 158.84 124.42) (end 158.85 124.41) (width 0.25) (layer F.Cu) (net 15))
 (segment (start 158.85 124.41) (end 159.92 124.41) (width 0.25) (layer F.Cu) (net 15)))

